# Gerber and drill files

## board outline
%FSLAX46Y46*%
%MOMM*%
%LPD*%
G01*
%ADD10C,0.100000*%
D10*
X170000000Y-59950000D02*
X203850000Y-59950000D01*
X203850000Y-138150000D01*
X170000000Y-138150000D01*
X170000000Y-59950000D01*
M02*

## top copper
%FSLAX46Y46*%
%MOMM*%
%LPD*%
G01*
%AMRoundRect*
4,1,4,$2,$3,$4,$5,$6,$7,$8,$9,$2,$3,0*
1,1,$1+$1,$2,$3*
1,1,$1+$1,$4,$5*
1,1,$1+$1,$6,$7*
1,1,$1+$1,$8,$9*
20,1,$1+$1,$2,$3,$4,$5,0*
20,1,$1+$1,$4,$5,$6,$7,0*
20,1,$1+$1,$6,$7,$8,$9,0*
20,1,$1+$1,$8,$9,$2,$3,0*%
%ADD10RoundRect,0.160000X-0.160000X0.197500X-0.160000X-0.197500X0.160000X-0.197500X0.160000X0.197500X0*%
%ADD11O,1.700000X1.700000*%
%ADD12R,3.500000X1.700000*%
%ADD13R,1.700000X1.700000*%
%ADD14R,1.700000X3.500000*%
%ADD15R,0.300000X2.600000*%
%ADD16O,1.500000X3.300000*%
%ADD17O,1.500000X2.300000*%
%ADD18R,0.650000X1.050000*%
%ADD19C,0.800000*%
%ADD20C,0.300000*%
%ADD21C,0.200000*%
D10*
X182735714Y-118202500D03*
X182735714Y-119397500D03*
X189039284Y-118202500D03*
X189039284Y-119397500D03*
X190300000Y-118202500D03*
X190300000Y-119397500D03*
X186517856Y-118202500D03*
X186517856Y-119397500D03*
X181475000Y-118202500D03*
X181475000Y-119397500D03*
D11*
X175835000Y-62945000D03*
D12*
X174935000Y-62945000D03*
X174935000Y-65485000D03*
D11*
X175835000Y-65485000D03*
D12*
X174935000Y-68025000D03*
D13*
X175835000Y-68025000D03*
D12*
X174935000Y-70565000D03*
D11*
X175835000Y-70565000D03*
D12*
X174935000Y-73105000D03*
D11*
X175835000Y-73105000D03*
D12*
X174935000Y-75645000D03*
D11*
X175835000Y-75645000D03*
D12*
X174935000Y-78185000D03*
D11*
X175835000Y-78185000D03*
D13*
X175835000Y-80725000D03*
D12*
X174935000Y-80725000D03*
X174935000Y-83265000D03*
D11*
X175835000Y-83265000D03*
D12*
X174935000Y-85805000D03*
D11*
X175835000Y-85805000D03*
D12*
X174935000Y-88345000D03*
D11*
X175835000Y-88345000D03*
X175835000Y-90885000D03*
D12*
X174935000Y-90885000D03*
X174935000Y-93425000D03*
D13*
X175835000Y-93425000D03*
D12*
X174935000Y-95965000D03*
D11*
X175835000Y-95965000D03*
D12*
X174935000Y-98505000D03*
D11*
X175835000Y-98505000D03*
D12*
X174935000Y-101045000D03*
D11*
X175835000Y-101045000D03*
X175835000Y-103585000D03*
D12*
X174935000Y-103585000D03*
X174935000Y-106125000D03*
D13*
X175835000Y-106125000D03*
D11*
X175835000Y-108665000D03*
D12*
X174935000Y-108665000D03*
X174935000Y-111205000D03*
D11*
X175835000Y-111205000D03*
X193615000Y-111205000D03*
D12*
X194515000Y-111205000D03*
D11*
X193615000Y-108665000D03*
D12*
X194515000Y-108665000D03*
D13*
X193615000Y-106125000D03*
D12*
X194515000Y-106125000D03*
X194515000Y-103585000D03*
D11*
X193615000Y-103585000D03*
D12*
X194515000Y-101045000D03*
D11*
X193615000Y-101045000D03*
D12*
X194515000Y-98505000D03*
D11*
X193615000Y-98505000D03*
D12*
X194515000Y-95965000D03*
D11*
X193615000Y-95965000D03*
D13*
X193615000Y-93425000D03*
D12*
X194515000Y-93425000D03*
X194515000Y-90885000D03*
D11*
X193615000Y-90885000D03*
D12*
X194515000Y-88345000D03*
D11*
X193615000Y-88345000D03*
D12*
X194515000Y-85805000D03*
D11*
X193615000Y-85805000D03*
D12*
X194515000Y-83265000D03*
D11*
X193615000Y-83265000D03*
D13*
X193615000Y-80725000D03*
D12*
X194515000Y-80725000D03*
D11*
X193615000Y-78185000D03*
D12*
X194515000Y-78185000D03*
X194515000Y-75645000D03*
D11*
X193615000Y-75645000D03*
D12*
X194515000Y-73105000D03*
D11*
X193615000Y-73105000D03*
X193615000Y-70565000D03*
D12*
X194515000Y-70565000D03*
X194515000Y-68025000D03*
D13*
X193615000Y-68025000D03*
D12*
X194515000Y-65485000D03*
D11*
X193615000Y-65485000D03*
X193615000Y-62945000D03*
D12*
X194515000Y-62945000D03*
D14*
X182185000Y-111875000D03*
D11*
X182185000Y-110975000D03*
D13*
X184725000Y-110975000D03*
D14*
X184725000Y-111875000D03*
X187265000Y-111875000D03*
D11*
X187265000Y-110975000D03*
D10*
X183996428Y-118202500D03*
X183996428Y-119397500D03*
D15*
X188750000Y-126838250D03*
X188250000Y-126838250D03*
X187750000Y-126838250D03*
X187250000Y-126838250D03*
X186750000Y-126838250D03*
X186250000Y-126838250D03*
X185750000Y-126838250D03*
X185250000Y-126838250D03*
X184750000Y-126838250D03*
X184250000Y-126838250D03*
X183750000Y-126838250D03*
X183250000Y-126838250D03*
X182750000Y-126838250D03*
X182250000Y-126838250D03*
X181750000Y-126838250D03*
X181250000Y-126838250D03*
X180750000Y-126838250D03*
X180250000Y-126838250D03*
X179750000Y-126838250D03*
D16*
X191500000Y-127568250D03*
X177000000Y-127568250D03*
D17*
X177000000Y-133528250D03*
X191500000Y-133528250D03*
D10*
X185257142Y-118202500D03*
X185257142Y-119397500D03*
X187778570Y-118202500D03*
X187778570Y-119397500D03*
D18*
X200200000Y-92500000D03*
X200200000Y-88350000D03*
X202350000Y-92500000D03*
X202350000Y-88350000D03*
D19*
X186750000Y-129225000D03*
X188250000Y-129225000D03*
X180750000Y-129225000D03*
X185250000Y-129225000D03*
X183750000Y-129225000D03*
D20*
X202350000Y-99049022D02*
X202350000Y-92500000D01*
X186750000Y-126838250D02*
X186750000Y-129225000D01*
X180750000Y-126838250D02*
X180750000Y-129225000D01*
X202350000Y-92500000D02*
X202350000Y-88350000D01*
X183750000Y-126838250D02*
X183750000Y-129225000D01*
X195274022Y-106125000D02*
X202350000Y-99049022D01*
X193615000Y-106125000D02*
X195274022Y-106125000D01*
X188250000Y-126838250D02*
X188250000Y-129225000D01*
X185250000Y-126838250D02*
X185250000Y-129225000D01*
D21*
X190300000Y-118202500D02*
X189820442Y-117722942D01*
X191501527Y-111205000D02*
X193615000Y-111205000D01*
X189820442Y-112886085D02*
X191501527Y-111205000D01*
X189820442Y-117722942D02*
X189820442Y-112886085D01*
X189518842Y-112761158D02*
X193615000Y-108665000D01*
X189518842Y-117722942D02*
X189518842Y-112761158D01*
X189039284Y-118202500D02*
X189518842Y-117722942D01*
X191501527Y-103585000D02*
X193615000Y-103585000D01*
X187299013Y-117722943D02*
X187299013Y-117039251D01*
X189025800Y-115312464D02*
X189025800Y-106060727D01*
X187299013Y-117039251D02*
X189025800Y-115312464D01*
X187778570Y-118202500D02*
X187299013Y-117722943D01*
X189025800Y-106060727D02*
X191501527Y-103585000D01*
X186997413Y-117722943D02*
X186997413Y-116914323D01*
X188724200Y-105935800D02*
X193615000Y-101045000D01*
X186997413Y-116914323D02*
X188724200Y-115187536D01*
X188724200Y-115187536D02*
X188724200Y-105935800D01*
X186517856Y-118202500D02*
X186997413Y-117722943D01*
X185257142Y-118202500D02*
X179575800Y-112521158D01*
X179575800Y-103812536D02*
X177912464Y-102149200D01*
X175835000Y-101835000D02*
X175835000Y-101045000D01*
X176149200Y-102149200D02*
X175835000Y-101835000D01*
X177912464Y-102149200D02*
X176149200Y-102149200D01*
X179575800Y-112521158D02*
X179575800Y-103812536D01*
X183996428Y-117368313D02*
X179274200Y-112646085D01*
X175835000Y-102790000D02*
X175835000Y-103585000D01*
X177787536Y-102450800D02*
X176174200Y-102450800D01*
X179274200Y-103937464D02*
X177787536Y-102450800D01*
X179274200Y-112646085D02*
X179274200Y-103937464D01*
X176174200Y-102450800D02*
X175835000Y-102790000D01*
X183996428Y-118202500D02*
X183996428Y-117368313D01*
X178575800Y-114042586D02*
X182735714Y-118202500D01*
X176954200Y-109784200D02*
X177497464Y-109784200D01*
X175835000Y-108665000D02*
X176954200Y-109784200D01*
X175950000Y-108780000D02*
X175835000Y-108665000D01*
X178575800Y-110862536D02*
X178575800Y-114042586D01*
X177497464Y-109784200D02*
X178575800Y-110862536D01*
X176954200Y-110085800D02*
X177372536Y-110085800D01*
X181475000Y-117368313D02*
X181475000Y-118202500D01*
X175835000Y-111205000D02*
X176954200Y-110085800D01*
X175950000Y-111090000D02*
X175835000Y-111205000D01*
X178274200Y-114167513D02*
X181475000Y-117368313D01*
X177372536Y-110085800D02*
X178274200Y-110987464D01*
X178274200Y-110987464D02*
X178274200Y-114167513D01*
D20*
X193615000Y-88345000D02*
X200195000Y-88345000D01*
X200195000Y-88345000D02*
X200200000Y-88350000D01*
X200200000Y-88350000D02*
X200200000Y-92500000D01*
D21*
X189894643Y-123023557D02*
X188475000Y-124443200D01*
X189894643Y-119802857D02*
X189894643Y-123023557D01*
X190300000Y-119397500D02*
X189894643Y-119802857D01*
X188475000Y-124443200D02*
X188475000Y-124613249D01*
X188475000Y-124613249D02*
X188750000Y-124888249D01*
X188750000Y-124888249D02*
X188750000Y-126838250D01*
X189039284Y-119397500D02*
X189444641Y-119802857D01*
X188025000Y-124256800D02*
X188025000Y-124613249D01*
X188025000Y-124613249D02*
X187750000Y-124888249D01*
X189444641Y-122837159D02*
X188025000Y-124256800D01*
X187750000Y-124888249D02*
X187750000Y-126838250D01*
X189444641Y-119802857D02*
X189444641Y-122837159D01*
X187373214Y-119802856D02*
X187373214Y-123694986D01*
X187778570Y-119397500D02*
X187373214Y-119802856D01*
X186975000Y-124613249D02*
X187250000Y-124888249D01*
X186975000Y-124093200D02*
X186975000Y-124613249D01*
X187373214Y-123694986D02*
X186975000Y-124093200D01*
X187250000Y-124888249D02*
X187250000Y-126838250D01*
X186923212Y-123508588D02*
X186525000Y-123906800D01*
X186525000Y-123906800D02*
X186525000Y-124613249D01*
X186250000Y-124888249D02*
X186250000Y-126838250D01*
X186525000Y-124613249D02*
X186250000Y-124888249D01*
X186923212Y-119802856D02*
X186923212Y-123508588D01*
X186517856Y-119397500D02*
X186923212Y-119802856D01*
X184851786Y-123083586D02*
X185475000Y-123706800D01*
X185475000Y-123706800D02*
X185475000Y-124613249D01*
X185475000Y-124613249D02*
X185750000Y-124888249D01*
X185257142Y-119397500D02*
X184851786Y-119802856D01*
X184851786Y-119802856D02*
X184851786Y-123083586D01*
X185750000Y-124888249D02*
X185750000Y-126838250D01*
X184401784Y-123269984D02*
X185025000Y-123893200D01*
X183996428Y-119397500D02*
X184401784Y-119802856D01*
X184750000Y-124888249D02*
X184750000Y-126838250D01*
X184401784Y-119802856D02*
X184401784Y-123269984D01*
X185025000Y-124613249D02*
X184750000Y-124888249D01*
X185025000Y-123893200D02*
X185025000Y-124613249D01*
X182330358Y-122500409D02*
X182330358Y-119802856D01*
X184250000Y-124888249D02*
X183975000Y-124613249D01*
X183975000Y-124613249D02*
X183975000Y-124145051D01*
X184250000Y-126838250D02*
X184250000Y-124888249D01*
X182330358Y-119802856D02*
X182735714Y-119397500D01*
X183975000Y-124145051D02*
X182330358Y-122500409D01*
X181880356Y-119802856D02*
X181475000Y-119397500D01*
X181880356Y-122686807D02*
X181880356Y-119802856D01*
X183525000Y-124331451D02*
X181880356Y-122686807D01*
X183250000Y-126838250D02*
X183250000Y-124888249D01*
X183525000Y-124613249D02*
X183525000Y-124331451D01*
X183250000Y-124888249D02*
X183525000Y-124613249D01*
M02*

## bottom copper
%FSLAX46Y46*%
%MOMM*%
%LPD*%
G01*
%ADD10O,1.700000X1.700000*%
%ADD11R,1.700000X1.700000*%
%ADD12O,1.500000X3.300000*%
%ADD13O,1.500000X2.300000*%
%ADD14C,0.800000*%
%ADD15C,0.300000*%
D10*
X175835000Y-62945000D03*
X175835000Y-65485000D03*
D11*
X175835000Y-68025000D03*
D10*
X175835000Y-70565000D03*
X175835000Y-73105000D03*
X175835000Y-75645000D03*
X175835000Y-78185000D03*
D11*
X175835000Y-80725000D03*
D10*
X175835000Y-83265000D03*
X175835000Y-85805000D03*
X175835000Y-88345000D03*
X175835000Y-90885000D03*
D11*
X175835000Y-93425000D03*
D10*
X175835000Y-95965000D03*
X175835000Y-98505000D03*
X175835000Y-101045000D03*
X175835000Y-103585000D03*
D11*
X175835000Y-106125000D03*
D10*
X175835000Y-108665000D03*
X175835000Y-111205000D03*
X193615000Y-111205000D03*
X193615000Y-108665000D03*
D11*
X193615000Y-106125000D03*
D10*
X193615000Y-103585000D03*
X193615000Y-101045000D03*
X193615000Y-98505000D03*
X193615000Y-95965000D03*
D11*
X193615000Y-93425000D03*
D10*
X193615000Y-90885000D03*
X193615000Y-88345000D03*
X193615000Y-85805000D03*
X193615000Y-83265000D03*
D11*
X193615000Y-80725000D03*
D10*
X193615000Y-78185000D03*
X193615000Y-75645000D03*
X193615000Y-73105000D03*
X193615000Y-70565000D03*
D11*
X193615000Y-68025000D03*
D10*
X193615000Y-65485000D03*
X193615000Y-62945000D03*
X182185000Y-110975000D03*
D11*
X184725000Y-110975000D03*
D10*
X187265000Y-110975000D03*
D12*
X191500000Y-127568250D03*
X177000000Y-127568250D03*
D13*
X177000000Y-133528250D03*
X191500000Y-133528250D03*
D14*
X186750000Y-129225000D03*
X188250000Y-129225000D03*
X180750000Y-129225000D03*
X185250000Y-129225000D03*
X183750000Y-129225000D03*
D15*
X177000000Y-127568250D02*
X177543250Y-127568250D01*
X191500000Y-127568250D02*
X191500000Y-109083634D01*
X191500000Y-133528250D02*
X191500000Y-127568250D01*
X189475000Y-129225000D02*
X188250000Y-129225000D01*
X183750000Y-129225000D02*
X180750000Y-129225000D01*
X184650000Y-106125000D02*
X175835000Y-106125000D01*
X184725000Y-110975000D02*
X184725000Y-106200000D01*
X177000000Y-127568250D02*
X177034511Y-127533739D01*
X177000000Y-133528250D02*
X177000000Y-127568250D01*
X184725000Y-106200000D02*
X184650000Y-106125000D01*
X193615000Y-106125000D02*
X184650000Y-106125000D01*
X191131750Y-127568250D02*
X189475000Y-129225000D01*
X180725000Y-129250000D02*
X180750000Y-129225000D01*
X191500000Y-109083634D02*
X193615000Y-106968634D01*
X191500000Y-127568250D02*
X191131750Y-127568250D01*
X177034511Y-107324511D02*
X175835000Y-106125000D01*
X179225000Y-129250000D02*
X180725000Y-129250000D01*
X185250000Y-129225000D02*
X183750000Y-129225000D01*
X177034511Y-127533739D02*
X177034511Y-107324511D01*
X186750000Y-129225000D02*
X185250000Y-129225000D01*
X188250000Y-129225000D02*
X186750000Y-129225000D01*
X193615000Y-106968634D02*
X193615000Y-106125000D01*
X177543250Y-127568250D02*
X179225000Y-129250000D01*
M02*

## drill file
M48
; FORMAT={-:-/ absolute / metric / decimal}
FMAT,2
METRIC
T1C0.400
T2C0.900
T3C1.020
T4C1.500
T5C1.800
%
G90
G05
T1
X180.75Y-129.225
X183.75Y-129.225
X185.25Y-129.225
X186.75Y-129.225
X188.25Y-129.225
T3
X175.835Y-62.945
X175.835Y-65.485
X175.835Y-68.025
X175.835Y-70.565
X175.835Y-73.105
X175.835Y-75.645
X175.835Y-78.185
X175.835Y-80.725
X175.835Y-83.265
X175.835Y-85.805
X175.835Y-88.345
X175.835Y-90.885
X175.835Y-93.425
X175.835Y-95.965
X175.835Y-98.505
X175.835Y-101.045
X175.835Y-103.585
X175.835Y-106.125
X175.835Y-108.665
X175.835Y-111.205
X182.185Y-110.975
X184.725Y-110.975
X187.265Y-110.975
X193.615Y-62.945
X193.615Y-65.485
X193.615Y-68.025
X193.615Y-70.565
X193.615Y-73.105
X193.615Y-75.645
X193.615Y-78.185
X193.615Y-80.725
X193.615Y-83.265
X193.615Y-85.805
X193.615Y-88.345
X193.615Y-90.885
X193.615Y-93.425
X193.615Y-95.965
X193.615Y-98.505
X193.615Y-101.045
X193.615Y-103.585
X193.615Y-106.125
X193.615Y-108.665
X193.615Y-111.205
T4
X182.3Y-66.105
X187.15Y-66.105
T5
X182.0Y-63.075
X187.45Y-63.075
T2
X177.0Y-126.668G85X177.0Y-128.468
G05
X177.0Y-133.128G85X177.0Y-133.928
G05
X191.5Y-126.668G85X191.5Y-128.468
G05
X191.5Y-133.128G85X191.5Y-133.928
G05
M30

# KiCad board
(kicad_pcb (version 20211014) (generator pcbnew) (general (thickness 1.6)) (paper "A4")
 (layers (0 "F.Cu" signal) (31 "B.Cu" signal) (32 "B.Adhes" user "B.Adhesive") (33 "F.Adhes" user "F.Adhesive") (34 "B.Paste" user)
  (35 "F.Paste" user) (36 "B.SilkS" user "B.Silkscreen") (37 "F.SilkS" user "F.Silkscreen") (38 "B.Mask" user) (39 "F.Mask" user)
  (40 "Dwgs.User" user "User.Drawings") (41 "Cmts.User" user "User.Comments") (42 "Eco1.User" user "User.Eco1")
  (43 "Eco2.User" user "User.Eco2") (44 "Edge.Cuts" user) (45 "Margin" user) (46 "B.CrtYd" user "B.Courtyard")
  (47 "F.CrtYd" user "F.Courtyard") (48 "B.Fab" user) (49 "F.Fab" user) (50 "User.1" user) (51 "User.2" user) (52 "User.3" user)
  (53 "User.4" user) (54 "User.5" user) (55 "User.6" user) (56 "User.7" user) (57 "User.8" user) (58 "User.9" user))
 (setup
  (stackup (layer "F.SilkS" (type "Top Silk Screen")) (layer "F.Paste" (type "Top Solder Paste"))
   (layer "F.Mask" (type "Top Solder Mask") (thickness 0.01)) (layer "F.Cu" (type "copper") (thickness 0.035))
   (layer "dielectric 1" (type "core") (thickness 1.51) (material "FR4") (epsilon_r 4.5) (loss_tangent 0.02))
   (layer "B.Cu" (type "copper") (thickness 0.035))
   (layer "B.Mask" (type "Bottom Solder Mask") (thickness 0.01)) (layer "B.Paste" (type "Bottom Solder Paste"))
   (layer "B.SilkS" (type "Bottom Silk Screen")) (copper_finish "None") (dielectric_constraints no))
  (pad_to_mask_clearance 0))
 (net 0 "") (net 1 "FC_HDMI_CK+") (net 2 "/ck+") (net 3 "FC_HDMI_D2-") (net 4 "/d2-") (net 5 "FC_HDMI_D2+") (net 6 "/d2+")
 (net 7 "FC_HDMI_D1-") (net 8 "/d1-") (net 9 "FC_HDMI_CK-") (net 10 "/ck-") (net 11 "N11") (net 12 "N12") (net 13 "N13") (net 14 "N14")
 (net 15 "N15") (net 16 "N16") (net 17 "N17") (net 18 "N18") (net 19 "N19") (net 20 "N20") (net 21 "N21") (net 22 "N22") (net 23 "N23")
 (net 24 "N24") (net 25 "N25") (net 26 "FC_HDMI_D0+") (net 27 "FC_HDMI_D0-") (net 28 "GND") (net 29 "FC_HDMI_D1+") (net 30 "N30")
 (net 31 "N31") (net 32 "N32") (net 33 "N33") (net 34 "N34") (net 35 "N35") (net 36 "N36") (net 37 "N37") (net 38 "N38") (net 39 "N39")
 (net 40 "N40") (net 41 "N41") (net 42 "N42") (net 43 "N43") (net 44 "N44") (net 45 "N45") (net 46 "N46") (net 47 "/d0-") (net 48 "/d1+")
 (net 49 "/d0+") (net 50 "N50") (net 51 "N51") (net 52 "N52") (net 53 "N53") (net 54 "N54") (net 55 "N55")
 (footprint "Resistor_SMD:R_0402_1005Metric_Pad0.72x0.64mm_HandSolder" (layer "F.Cu") (at 182.735714 118.8 -90)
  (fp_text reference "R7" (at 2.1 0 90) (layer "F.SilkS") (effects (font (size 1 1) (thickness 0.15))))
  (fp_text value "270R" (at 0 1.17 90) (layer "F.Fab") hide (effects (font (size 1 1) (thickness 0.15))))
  (pad "1" smd roundrect locked (at -0.5975 0 270) (size 0.715 0.64) (layers "F.Cu" "F.Paste" "F.Mask") (roundrect_rratio 0.25)
   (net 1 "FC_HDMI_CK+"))
  (pad "2" smd roundrect locked (at 0.5975 0 270) (size 0.715 0.64) (layers "F.Cu" "F.Paste" "F.Mask") (roundrect_rratio 0.25)
   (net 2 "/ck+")))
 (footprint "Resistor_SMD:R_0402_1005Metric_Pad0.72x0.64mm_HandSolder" (layer "F.Cu") (at 189.039284 118.8 -90)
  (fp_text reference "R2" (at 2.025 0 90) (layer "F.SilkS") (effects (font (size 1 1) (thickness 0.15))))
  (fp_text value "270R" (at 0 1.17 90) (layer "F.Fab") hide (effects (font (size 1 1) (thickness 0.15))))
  (pad "1" smd roundrect locked (at -0.5975 0 270) (size 0.715 0.64) (layers "F.Cu" "F.Paste" "F.Mask") (roundrect_rratio 0.25)
   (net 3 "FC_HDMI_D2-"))
  (pad "2" smd roundrect locked (at 0.5975 0 270) (size 0.715 0.64) (layers "F.Cu" "F.Paste" "F.Mask") (roundrect_rratio 0.25)
   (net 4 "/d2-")))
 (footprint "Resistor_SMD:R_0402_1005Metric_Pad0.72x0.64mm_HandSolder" (layer "F.Cu") (at 190.3 118.8 -90)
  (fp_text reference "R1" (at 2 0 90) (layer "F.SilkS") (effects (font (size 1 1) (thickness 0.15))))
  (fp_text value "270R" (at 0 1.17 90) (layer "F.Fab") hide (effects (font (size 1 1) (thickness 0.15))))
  (pad "1" smd roundrect locked (at -0.5975 0 270) (size 0.715 0.64) (layers "F.Cu" "F.Paste" "F.Mask") (roundrect_rratio 0.25)
   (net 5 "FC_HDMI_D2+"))
  (pad "2" smd roundrect locked (at 0.5975 0 270) (size 0.715 0.64) (layers "F.Cu" "F.Paste" "F.Mask") (roundrect_rratio 0.25)
   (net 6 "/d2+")))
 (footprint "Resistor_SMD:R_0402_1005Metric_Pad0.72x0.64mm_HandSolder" (layer "F.Cu") (at 186.517856 118.8 -90)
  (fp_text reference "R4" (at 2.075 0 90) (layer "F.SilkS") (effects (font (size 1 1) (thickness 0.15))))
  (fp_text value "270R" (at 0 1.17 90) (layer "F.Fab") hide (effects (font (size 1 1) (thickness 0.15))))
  (pad "1" smd roundrect locked (at -0.5975 0 270) (size 0.715 0.64) (layers "F.Cu" "F.Paste" "F.Mask") (roundrect_rratio 0.25)
   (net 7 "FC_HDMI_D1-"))
  (pad "2" smd roundrect locked (at 0.5975 0 270) (size 0.715 0.64) (layers "F.Cu" "F.Paste" "F.Mask") (roundrect_rratio 0.25)
   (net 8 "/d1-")))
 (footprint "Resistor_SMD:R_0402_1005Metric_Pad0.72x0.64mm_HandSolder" (layer "F.Cu") (at 181.475 118.8 -90)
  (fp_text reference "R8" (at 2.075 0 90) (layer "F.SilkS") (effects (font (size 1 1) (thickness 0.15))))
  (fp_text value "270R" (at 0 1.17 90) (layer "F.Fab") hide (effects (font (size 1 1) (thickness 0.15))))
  (pad "1" smd roundrect locked (at -0.5975 0 270) (size 0.715 0.64) (layers "F.Cu" "F.Paste" "F.Mask") (roundrect_rratio 0.25)
   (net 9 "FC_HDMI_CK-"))
  (pad "2" smd roundrect locked (at 0.5975 0 270) (size 0.715 0.64) (layers "F.Cu" "F.Paste" "F.Mask") (roundrect_rratio 0.25)
   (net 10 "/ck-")))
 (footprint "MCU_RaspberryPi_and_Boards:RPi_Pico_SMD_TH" (layer "F.Cu") (at 184.725 87.075)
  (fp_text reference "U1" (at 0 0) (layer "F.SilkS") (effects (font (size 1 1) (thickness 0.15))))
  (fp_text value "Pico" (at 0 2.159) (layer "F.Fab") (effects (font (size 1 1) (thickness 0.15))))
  (pad "" np_thru_hole oval locked (at -2.725 -24) (size 1.8 1.8) (drill 1.8) (layers *.Cu *.Mask))
  (pad "" np_thru_hole oval locked (at 2.725 -24) (size 1.8 1.8) (drill 1.8) (layers *.Cu *.Mask))
  (pad "" np_thru_hole oval locked (at 2.425 -20.97) (size 1.5 1.5) (drill 1.5) (layers *.Cu *.Mask))
  (pad "" np_thru_hole oval locked (at -2.425 -20.97) (size 1.5 1.5) (drill 1.5) (layers *.Cu *.Mask))
  (pad "1" thru_hole oval locked (at -8.89 -24.13) (size 1.7 1.7) (drill 1.02) (layers *.Cu *.Mask) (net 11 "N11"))
  (pad "1" smd rect locked (at -8.89 -24.13) (size 3.5 1.7) (drill (offset -0.9 0)) (layers "F.Cu" "F.Mask") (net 11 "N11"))
  (pad "2" smd rect locked (at -8.89 -21.59) (size 3.5 1.7) (drill (offset -0.9 0)) (layers "F.Cu" "F.Mask") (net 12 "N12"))
  (pad "2" thru_hole oval locked (at -8.89 -21.59) (size 1.7 1.7) (drill 1.02) (layers *.Cu *.Mask) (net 12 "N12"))
  (pad "3" smd rect locked (at -8.89 -19.05) (size 3.5 1.7) (drill (offset -0.9 0)) (layers "F.Cu" "F.Mask") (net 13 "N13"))
  (pad "3" thru_hole rect locked (at -8.89 -19.05) (size 1.7 1.7) (drill 1.02) (layers *.Cu *.Mask) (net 13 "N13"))
  (pad "4" smd rect locked (at -8.89 -16.51) (size 3.5 1.7) (drill (offset -0.9 0)) (layers "F.Cu" "F.Mask") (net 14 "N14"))
  (pad "4" thru_hole oval locked (at -8.89 -16.51) (size 1.7 1.7) (drill 1.02) (layers *.Cu *.Mask) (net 14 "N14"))
  (pad "5" smd rect locked (at -8.89 -13.97) (size 3.5 1.7) (drill (offset -0.9 0)) (layers "F.Cu" "F.Mask") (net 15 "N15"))
  (pad "5" thru_hole oval locked (at -8.89 -13.97) (size 1.7 1.7) (drill 1.02) (layers *.Cu *.Mask) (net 15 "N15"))
  (pad "6" smd rect locked (at -8.89 -11.43) (size 3.5 1.7) (drill (offset -0.9 0)) (layers "F.Cu" "F.Mask") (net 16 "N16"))
  (pad "6" thru_hole oval locked (at -8.89 -11.43) (size 1.7 1.7) (drill 1.02) (layers *.Cu *.Mask) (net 16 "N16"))
  (pad "7" smd rect locked (at -8.89 -8.89) (size 3.5 1.7) (drill (offset -0.9 0)) (layers "F.Cu" "F.Mask") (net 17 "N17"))
  (pad "7" thru_hole oval locked (at -8.89 -8.89) (size 1.7 1.7) (drill 1.02) (layers *.Cu *.Mask) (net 17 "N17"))
  (pad "8" thru_hole rect locked (at -8.89 -6.35) (size 1.7 1.7) (drill 1.02) (layers *.Cu *.Mask) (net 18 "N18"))
  (pad "8" smd rect locked (at -8.89 -6.35) (size 3.5 1.7) (drill (offset -0.9 0)) (layers "F.Cu" "F.Mask") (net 18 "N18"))
  (pad "9" smd rect locked (at -8.89 -3.81) (size 3.5 1.7) (drill (offset -0.9 0)) (layers "F.Cu" "F.Mask") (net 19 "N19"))
  (pad "9" thru_hole oval locked (at -8.89 -3.81) (size 1.7 1.7) (drill 1.02) (layers *.Cu *.Mask) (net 19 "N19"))
  (pad "10" smd rect locked (at -8.89 -1.27) (size 3.5 1.7) (drill (offset -0.9 0)) (layers "F.Cu" "F.Mask") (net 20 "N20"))
  (pad "10" thru_hole oval locked (at -8.89 -1.27) (size 1.7 1.7) (drill 1.02) (layers *.Cu *.Mask) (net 20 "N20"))
  (pad "11" smd rect locked (at -8.89 1.27) (size 3.5 1.7) (drill (offset -0.9 0)) (layers "F.Cu" "F.Mask") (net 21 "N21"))
  (pad "11" thru_hole oval locked (at -8.89 1.27) (size 1.7 1.7) (drill 1.02) (layers *.Cu *.Mask) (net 21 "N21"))
  (pad "12" thru_hole oval locked (at -8.89 3.81) (size 1.7 1.7) (drill 1.02) (layers *.Cu *.Mask) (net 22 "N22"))
  (pad "12" smd rect locked (at -8.89 3.81) (size 3.5 1.7) (drill (offset -0.9 0)) (layers "F.Cu" "F.Mask") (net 22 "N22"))
  (pad "13" smd rect locked (at -8.89 6.35) (size 3.5 1.7) (drill (offset -0.9 0)) (layers "F.Cu" "F.Mask") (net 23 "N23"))
  (pad "13" thru_hole rect locked (at -8.89 6.35) (size 1.7 1.7) (drill 1.02) (layers *.Cu *.Mask) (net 23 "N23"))
  (pad "14" smd rect locked (at -8.89 8.89) (size 3.5 1.7) (drill (offset -0.9 0)) (layers "F.Cu" "F.Mask") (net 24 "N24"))
  (pad "14" thru_hole oval locked (at -8.89 8.89) (size 1.7 1.7) (drill 1.02) (layers *.Cu *.Mask) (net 24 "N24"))
  (pad "15" smd rect locked (at -8.89 11.43) (size 3.5 1.7) (drill (offset -0.9 0)) (layers "F.Cu" "F.Mask") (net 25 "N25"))
  (pad "15" thru_hole oval locked (at -8.89 11.43) (size 1.7 1.7) (drill 1.02) (layers *.Cu *.Mask) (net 25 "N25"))
  (pad "16" smd rect locked (at -8.89 13.97) (size 3.5 1.7) (drill (offset -0.9 0)) (layers "F.Cu" "F.Mask") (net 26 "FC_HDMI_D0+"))
  (pad "16" thru_hole oval locked (at -8.89 13.97) (size 1.7 1.7) (drill 1.02) (layers *.Cu *.Mask) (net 26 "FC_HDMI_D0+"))
  (pad "17" thru_hole oval locked (at -8.89 16.51) (size 1.7 1.7) (drill 1.02) (layers *.Cu *.Mask) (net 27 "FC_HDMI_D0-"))
  (pad "17" smd rect locked (at -8.89 16.51) (size 3.5 1.7) (drill (offset -0.9 0)) (layers "F.Cu" "F.Mask") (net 27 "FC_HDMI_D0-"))
  (pad "18" smd rect locked (at -8.89 19.05) (size 3.5 1.7) (drill (offset -0.9 0)) (layers "F.Cu" "F.Mask") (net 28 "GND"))
  (pad "18" thru_hole rect locked (at -8.89 19.05) (size 1.7 1.7) (drill 1.02) (layers *.Cu *.Mask) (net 28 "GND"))
  (pad "19" thru_hole oval locked (at -8.89 21.59) (size 1.7 1.7) (drill 1.02) (layers *.Cu *.Mask) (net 1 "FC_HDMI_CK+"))
  (pad "19" smd rect locked (at -8.89 21.59) (size 3.5 1.7) (drill (offset -0.9 0)) (layers "F.Cu" "F.Mask") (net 1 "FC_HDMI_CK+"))
  (pad "20" smd rect locked (at -8.89 24.13) (size 3.5 1.7) (drill (offset -0.9 0)) (layers "F.Cu" "F.Mask") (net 9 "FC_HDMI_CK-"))
  (pad "20" thru_hole oval locked (at -8.89 24.13) (size 1.7 1.7) (drill 1.02) (layers *.Cu *.Mask) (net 9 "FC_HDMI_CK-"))
  (pad "21" thru_hole oval locked (at 8.89 24.13) (size 1.7 1.7) (drill 1.02) (layers *.Cu *.Mask) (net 5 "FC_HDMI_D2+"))
  (pad "21" smd rect locked (at 8.89 24.13) (size 3.5 1.7) (drill (offset 0.9 0)) (layers "F.Cu" "F.Mask") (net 5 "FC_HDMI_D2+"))
  (pad "22" thru_hole oval locked (at 8.89 21.59) (size 1.7 1.7) (drill 1.02) (layers *.Cu *.Mask) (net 3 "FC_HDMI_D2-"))
  (pad "22" smd rect locked (at 8.89 21.59) (size 3.5 1.7) (drill (offset 0.9 0)) (layers "F.Cu" "F.Mask") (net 3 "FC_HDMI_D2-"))
  (pad "23" thru_hole rect locked (at 8.89 19.05) (size 1.7 1.7) (drill 1.02) (layers *.Cu *.Mask) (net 28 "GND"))
  (pad "23" smd rect locked (at 8.89 19.05) (size 3.5 1.7) (drill (offset 0.9 0)) (layers "F.Cu" "F.Mask") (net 28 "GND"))
  (pad "24" smd rect locked (at 8.89 16.51) (size 3.5 1.7) (drill (offset 0.9 0)) (layers "F.Cu" "F.Mask") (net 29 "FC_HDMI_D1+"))
  (pad "24" thru_hole oval locked (at 8.89 16.51) (size 1.7 1.7) (drill 1.02) (layers *.Cu *.Mask) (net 29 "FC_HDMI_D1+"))
  (pad "25" smd rect locked (at 8.89 13.97) (size 3.5 1.7) (drill (offset 0.9 0)) (layers "F.Cu" "F.Mask") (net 7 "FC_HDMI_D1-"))
  (pad "25" thru_hole oval locked (at 8.89 13.97) (size 1.7 1.7) (drill 1.02) (layers *.Cu *.Mask) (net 7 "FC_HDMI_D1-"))
  (pad "26" smd rect locked (at 8.89 11.43) (size 3.5 1.7) (drill (offset 0.9 0)) (layers "F.Cu" "F.Mask") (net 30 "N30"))
  (pad "26" thru_hole oval locked (at 8.89 11.43) (size 1.7 1.7) (drill 1.02) (layers *.Cu *.Mask) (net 30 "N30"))
  (pad "27" smd rect locked (at 8.89 8.89) (size 3.5 1.7) (drill (offset 0.9 0)) (layers "F.Cu" "F.Mask") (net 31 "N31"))
  (pad "27" thru_hole oval locked (at 8.89 8.89) (size 1.7 1.7) (drill 1.02) (layers *.Cu *.Mask) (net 31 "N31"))
  (pad "28" thru_hole rect locked (at 8.89 6.35) (size 1.7 1.7) (drill 1.02) (layers *.Cu *.Mask) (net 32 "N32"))
  (pad "28" smd rect locked (at 8.89 6.35) (size 3.5 1.7) (drill (offset 0.9 0)) (layers "F.Cu" "F.Mask") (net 32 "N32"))
  (pad "29" smd rect locked (at 8.89 3.81) (size 3.5 1.7) (drill (offset 0.9 0)) (layers "F.Cu" "F.Mask") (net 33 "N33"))
  (pad "29" thru_hole oval locked (at 8.89 3.81) (size 1.7 1.7) (drill 1.02) (layers *.Cu *.Mask) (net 33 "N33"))
  (pad "30" smd rect locked (at 8.89 1.27) (size 3.5 1.7) (drill (offset 0.9 0)) (layers "F.Cu" "F.Mask") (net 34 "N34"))
  (pad "30" thru_hole oval locked (at 8.89 1.27) (size 1.7 1.7) (drill 1.02) (layers *.Cu *.Mask) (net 34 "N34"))
  (pad "31" smd rect locked (at 8.89 -1.27) (size 3.5 1.7) (drill (offset 0.9 0)) (layers "F.Cu" "F.Mask") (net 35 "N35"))
  (pad "31" thru_hole oval locked (at 8.89 -1.27) (size 1.7 1.7) (drill 1.02) (layers *.Cu *.Mask) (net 35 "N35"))
  (pad "32" smd rect locked (at 8.89 -3.81) (size 3.5 1.7) (drill (offset 0.9 0)) (layers "F.Cu" "F.Mask") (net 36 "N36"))
  (pad "32" thru_hole oval locked (at 8.89 -3.81) (size 1.7 1.7) (drill 1.02) (layers *.Cu *.Mask) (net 36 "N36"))
  (pad "33" thru_hole rect locked (at 8.89 -6.35) (size 1.7 1.7) (drill 1.02) (layers *.Cu *.Mask) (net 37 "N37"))
  (pad "33" smd rect locked (at 8.89 -6.35) (size 3.5 1.7) (drill (offset 0.9 0)) (layers "F.Cu" "F.Mask") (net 37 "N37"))
  (pad "34" thru_hole oval locked (at 8.89 -8.89) (size 1.7 1.7) (drill 1.02) (layers *.Cu *.Mask) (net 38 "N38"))
  (pad "34" smd rect locked (at 8.89 -8.89) (size 3.5 1.7) (drill (offset 0.9 0)) (layers "F.Cu" "F.Mask") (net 38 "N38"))
  (pad "35" smd rect locked (at 8.89 -11.43) (size 3.5 1.7) (drill (offset 0.9 0)) (layers "F.Cu" "F.Mask") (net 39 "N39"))
  (pad "35" thru_hole oval locked (at 8.89 -11.43) (size 1.7 1.7) (drill 1.02) (layers *.Cu *.Mask) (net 39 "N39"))
  (pad "36" smd rect locked (at 8.89 -13.97) (size 3.5 1.7) (drill (offset 0.9 0)) (layers "F.Cu" "F.Mask") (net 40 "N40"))
  (pad "36" thru_hole oval locked (at 8.89 -13.97) (size 1.7 1.7) (drill 1.02) (layers *.Cu *.Mask) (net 40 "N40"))
  (pad "37" thru_hole oval locked (at 8.89 -16.51) (size 1.7 1.7) (drill 1.02) (layers *.Cu *.Mask) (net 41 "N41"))
  (pad "37" smd rect locked (at 8.89 -16.51) (size 3.5 1.7) (drill (offset 0.9 0)) (layers "F.Cu" "F.Mask") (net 41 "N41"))
  (pad "38" smd rect locked (at 8.89 -19.05) (size 3.5 1.7) (drill (offset 0.9 0)) (layers "F.Cu" "F.Mask") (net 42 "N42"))
  (pad "38" thru_hole rect locked (at 8.89 -19.05) (size 1.7 1.7) (drill 1.02) (layers *.Cu *.Mask) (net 42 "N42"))
  (pad "39" smd rect locked (at 8.89 -21.59) (size 3.5 1.7) (drill (offset 0.9 0)) (layers "F.Cu" "F.Mask") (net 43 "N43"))
  (pad "39" thru_hole oval locked (at 8.89 -21.59) (size 1.7 1.7) (drill 1.02) (layers *.Cu *.Mask) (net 43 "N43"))
  (pad "40" thru_hole oval locked (at 8.89 -24.13) (size 1.7 1.7) (drill 1.02) (layers *.Cu *.Mask) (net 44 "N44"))
  (pad "40" smd rect locked (at 8.89 -24.13) (size 3.5 1.7) (drill (offset 0.9 0)) (layers "F.Cu" "F.Mask") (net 44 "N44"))
  (pad "41" smd rect locked (at -2.54 23.9 90) (size 3.5 1.7) (drill (offset -0.9 0)) (layers "F.Cu" "F.Mask") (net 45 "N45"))
  (pad "41" thru_hole oval locked (at -2.54 23.9) (size 1.7 1.7) (drill 1.02) (layers *.Cu *.Mask) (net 45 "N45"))
  (pad "42" thru_hole rect locked (at 0 23.9) (size 1.7 1.7) (drill 1.02) (layers *.Cu *.Mask) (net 28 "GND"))
  (pad "42" smd rect locked (at 0 23.9 90) (size 3.5 1.7) (drill (offset -0.9 0)) (layers "F.Cu" "F.Mask") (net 28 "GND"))
  (pad "43" smd rect locked (at 2.54 23.9 90) (size 3.5 1.7) (drill (offset -0.9 0)) (layers "F.Cu" "F.Mask") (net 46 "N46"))
  (pad "43" thru_hole oval locked (at 2.54 23.9) (size 1.7 1.7) (drill 1.02) (layers *.Cu *.Mask) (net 46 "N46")))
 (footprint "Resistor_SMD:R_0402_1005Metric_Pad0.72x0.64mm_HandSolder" (layer "F.Cu") (at 183.996428 118.8 -90)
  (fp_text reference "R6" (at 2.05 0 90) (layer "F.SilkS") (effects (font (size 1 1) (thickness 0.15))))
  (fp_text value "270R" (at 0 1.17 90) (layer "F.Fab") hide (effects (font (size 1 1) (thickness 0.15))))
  (pad "1" smd roundrect locked (at -0.5975 0 270) (size 0.715 0.64) (layers "F.Cu" "F.Paste" "F.Mask") (roundrect_rratio 0.25)
   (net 27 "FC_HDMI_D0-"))
  (pad "2" smd roundrect locked (at 0.5975 0 270) (size 0.715 0.64) (layers "F.Cu" "F.Paste" "F.Mask") (roundrect_rratio 0.25)
   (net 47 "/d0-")))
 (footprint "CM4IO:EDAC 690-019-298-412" (layer "F.Cu") (at 184.25 127.56825)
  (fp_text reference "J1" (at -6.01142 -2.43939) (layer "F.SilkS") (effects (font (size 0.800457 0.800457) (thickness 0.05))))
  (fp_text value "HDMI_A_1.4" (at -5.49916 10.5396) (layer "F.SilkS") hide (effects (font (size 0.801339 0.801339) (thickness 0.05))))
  (pad "1" smd rect (at 4.5 -0.73 90) (size 2.6 0.3) (layers "F.Cu" "F.Paste" "F.Mask") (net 6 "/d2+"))
  (pad "2" smd rect (at 4 -0.73 90) (size 2.6 0.3) (layers "F.Cu" "F.Paste" "F.Mask") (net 28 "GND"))
  (pad "3" smd rect (at 3.5 -0.73 90) (size 2.6 0.3) (layers "F.Cu" "F.Paste" "F.Mask") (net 4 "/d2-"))
  (pad "4" smd rect (at 3 -0.73 90) (size 2.6 0.3) (layers "F.Cu" "F.Paste" "F.Mask") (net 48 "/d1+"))
  (pad "5" smd rect (at 2.5 -0.73 90) (size 2.6 0.3) (layers "F.Cu" "F.Paste" "F.Mask") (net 28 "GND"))
  (pad "6" smd rect (at 2 -0.73 90) (size 2.6 0.3) (layers "F.Cu" "F.Paste" "F.Mask") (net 8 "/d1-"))
  (pad "7" smd rect (at 1.5 -0.73 90) (size 2.6 0.3) (layers "F.Cu" "F.Paste" "F.Mask") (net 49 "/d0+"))
  (pad "8" smd rect (at 1 -0.73 90) (size 2.6 0.3) (layers "F.Cu" "F.Paste" "F.Mask") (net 28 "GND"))
  (pad "9" smd rect (at 0.5 -0.73 90) (size 2.6 0.3) (layers "F.Cu" "F.Paste" "F.Mask") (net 47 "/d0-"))
  (pad "10" smd rect (at 0 -0.73 90) (size 2.6 0.3) (layers "F.Cu" "F.Paste" "F.Mask") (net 2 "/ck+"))
  (pad "11" smd rect (at -0.5 -0.73 90) (size 2.6 0.3) (layers "F.Cu" "F.Paste" "F.Mask") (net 28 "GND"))
  (pad "12" smd rect (at -1 -0.73 90) (size 2.6 0.3) (layers "F.Cu" "F.Paste" "F.Mask") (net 10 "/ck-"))
  (pad "13" smd rect (at -1.5 -0.73 90) (size 2.6 0.3) (layers "F.Cu" "F.Paste" "F.Mask") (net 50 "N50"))
  (pad "14" smd rect (at -2 -0.73 90) (size 2.6 0.3) (layers "F.Cu" "F.Paste" "F.Mask") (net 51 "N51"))
  (pad "15" smd rect (at -2.5 -0.73 90) (size 2.6 0.3) (layers "F.Cu" "F.Paste" "F.Mask") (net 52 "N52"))
  (pad "16" smd rect (at -3 -0.73 90) (size 2.6 0.3) (layers "F.Cu" "F.Paste" "F.Mask") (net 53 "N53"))
  (pad "17" smd rect (at -3.5 -0.73 90) (size 2.6 0.3) (layers "F.Cu" "F.Paste" "F.Mask") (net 28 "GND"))
  (pad "18" smd rect (at -4 -0.73 90) (size 2.6 0.3) (layers "F.Cu" "F.Paste" "F.Mask") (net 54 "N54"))
  (pad "19" smd rect (at -4.5 -0.73 90) (size 2.6 0.3) (layers "F.Cu" "F.Paste" "F.Mask") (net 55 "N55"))
  (pad "SH1" thru_hole oval (at 7.25 0) (size 1.5 3.3) (drill oval 0.9 2.7) (layers *.Cu *.Mask) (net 28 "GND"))
  (pad "SH2" thru_hole oval (at -7.25 0) (size 1.5 3.3) (drill oval 0.9 2.7) (layers *.Cu *.Mask) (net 28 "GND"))
  (pad "SH3" thru_hole oval (at -7.25 5.96) (size 1.5 2.3) (drill oval 0.9 1.7) (layers *.Cu *.Mask) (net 28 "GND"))
  (pad "SH4" thru_hole oval (at 7.25 5.96) (size 1.5 2.3) (drill oval 0.9 1.7) (layers *.Cu *.Mask) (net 28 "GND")))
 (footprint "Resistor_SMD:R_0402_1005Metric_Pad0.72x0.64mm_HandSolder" (layer "F.Cu") (at 185.257142 118.8 -90)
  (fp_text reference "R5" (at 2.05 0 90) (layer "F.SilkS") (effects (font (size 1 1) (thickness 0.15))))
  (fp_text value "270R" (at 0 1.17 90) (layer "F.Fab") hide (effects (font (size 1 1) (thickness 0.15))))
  (pad "1" smd roundrect locked (at -0.5975 0 270) (size 0.715 0.64) (layers "F.Cu" "F.Paste" "F.Mask") (roundrect_rratio 0.25)
   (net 26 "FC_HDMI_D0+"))
  (pad "2" smd roundrect locked (at 0.5975 0 270) (size 0.715 0.64) (layers "F.Cu" "F.Paste" "F.Mask") (roundrect_rratio 0.25)
   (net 49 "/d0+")))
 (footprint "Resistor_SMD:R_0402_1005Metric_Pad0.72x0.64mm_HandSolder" (layer "F.Cu") (at 187.77857 118.8 -90)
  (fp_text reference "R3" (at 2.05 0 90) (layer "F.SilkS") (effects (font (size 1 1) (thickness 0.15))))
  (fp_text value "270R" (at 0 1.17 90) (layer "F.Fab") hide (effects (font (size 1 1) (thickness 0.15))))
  (pad "1" smd roundrect locked (at -0.5975 0 270) (size 0.715 0.64) (layers "F.Cu" "F.Paste" "F.Mask") (roundrect_rratio 0.25)
   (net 29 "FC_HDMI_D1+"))
  (pad "2" smd roundrect locked (at 0.5975 0 270) (size 0.715 0.64) (layers "F.Cu" "F.Paste" "F.Mask") (roundrect_rratio 0.25)
   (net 48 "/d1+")))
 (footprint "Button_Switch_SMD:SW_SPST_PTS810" (layer "F.Cu") (at 201.275 90.425 90)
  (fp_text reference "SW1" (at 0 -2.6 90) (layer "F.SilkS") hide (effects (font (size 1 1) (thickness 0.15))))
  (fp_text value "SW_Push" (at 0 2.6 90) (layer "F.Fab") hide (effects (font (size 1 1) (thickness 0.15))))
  (pad "1" smd rect locked (at -2.075 -1.075 90) (size 1.05 0.65) (layers "F.Cu" "F.Paste" "F.Mask") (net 34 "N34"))
  (pad "1" smd rect locked (at 2.075 -1.075 90) (size 1.05 0.65) (layers "F.Cu" "F.Paste" "F.Mask") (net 34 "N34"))
  (pad "2" smd rect locked (at -2.075 1.075 90) (size 1.05 0.65) (layers "F.Cu" "F.Paste" "F.Mask") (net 28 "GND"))
  (pad "2" smd rect locked (at 2.075 1.075 90) (size 1.05 0.65) (layers "F.Cu" "F.Paste" "F.Mask") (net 28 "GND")))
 (gr_rect (start 170 59.95) (end 203.85 138.15) (layer "Edge.Cuts") (width 0.1) (fill none))
 (segment (start 202.35 99.049022) (end 202.35 92.5) (width 0.3) (layer "F.Cu") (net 28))
 (segment (start 186.75 126.83825) (end 186.75 129.225) (width 0.3) (layer "F.Cu") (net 28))
 (segment (start 180.75 126.83825) (end 180.75 129.225) (width 0.3) (layer "F.Cu") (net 28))
 (segment (start 202.35 92.5) (end 202.35 88.35) (width 0.3) (layer "F.Cu") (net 28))
 (segment (start 183.75 126.83825) (end 183.75 129.225) (width 0.3) (layer "F.Cu") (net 28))
 (segment (start 195.274022 106.125) (end 202.35 99.049022) (width 0.3) (layer "F.Cu") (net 28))
 (segment (start 193.615 106.125) (end 195.274022 106.125) (width 0.3) (layer "F.Cu") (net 28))
 (segment (start 188.25 126.83825) (end 188.25 129.225) (width 0.3) (layer "F.Cu") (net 28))
 (segment (start 185.25 126.83825) (end 185.25 129.225) (width 0.3) (layer "F.Cu") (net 28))
 (via (at 186.75 129.225) (size 0.8) (drill 0.4) (layers "F.Cu" "B.Cu") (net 28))
 (via (at 188.25 129.225) (size 0.8) (drill 0.4) (layers "F.Cu" "B.Cu") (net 28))
 (via (at 180.75 129.225) (size 0.8) (drill 0.4) (layers "F.Cu" "B.Cu") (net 28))
 (via (at 185.25 129.225) (size 0.8) (drill 0.4) (layers "F.Cu" "B.Cu") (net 28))
 (via (at 183.75 129.225) (size 0.8) (drill 0.4) (layers "F.Cu" "B.Cu") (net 28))
 (segment (start 177 127.56825) (end 177.54325 127.56825) (width 0.3) (layer "B.Cu") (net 28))
 (segment (start 191.5 127.56825) (end 191.5 109.083634) (width 0.3) (layer "B.Cu") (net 28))
 (segment (start 191.5 133.52825) (end 191.5 127.56825) (width 0.3) (layer "B.Cu") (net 28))
 (segment (start 189.475 129.225) (end 188.25 129.225) (width 0.3) (layer "B.Cu") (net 28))
 (segment (start 183.75 129.225) (end 180.75 129.225) (width 0.3) (layer "B.Cu") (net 28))
 (segment (start 184.65 106.125) (end 175.835 106.125) (width 0.3) (layer "B.Cu") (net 28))
 (segment (start 184.725 110.975) (end 184.725 106.2) (width 0.3) (layer "B.Cu") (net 28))
 (segment (start 177 127.56825) (end 177.034511 127.533739) (width 0.3) (layer "B.Cu") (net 28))
 (segment (start 177 133.52825) (end 177 127.56825) (width 0.3) (layer "B.Cu") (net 28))
 (segment (start 184.725 106.2) (end 184.65 106.125) (width 0.3) (layer "B.Cu") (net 28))
 (segment (start 193.615 106.125) (end 184.65 106.125) (width 0.3) (layer "B.Cu") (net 28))
 (segment (start 191.13175 127.56825) (end 189.475 129.225) (width 0.3) (layer "B.Cu") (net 28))
 (segment (start 180.725 129.25) (end 180.75 129.225) (width 0.3) (layer "B.Cu") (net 28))
 (segment (start 191.5 109.083634) (end 193.615 106.968634) (width 0.3) (layer "B.Cu") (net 28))
 (segment (start 191.5 127.56825) (end 191.13175 127.56825) (width 0.3) (layer "B.Cu") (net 28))
 (segment (start 177.034511 107.324511) (end 175.835 106.125) (width 0.3) (layer "B.Cu") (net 28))
 (segment (start 179.225 129.25) (end 180.725 129.25) (width 0.3) (layer "B.Cu") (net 28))
 (segment (start 185.25 129.225) (end 183.75 129.225) (width 0.3) (layer "B.Cu") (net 28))
 (segment (start 177.034511 127.533739) (end 177.034511 107.324511) (width 0.3) (layer "B.Cu") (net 28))
 (segment (start 186.75 129.225) (end 185.25 129.225) (width 0.3) (layer "B.Cu") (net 28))
 (segment (start 188.25 129.225) (end 186.75 129.225) (width 0.3) (layer "B.Cu") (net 28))
 (segment (start 193.615 106.968634) (end 193.615 106.125) (width 0.3) (layer "B.Cu") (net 28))
 (segment (start 177.54325 127.56825) (end 179.225 129.25) (width 0.3) (layer "B.Cu") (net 28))
 (segment (start 190.3 118.2025) (end 189.820442 117.722942) (width 0.2) (layer "F.Cu") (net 5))
 (segment (start 191.501527 111.205) (end 193.615 111.205) (width 0.2) (layer "F.Cu") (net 5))
 (segment (start 189.820442 112.886085) (end 191.501527 111.205) (width 0.2) (layer "F.Cu") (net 5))
 (segment (start 189.820442 117.722942) (end 189.820442 112.886085) (width 0.2) (layer "F.Cu") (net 5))
 (segment (start 189.518842 112.761158) (end 193.615 108.665) (width 0.2) (layer "F.Cu") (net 3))
 (segment (start 189.518842 117.722942) (end 189.518842 112.761158) (width 0.2) (layer "F.Cu") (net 3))
 (segment (start 189.039284 118.2025) (end 189.518842 117.722942) (width 0.2) (layer "F.Cu") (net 3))
 (segment (start 191.501527 103.585) (end 193.615 103.585) (width 0.2) (layer "F.Cu") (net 29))
 (segment (start 187.299013 117.722943) (end 187.299013 117.039251) (width 0.2) (layer "F.Cu") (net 29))
 (segment (start 189.0258 115.312464) (end 189.0258 106.060727) (width 0.2) (layer "F.Cu") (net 29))
 (segment (start 187.299013 117.039251) (end 189.0258 115.312464) (width 0.2) (layer "F.Cu") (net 29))
 (segment (start 187.77857 118.2025) (end 187.299013 117.722943) (width 0.2) (layer "F.Cu") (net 29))
 (segment (start 189.0258 106.060727) (end 191.501527 103.585) (width 0.2) (layer "F.Cu") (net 29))
 (segment (start 186.997413 117.722943) (end 186.997413 116.914323) (width 0.2) (layer "F.Cu") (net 7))
 (segment (start 188.7242 105.9358) (end 193.615 101.045) (width 0.2) (layer "F.Cu") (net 7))
 (segment (start 186.997413 116.914323) (end 188.7242 115.187536) (width 0.2) (layer "F.Cu") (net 7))
 (segment (start 188.7242 115.187536) (end 188.7242 105.9358) (width 0.2) (layer "F.Cu") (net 7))
 (segment (start 186.517856 118.2025) (end 186.997413 117.722943) (width 0.2) (layer "F.Cu") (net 7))
 (segment (start 185.257142 118.2025) (end 179.5758 112.521158) (width 0.2) (layer "F.Cu") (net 26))
 (segment (start 179.5758 103.812536) (end 177.912464 102.1492) (width 0.2) (layer "F.Cu") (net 26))
 (segment (start 175.835 101.835) (end 175.835 101.045) (width 0.2) (layer "F.Cu") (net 26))
 (segment (start 176.1492 102.1492) (end 175.835 101.835) (width 0.2) (layer "F.Cu") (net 26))
 (segment (start 177.912464 102.1492) (end 176.1492 102.1492) (width 0.2) (layer "F.Cu") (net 26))
 (segment (start 179.5758 112.521158) (end 179.5758 103.812536) (width 0.2) (layer "F.Cu") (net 26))
 (segment (start 183.996428 117.368313) (end 179.2742 112.646085) (width 0.2) (layer "F.Cu") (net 27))
 (segment (start 175.835 102.79) (end 175.835 103.585) (width 0.2) (layer "F.Cu") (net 27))
 (segment (start 177.787536 102.4508) (end 176.1742 102.4508) (width 0.2) (layer "F.Cu") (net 27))
 (segment (start 179.2742 103.937464) (end 177.787536 102.4508) (width 0.2) (layer "F.Cu") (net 27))
 (segment (start 179.2742 112.646085) (end 179.2742 103.937464) (width 0.2) (layer "F.Cu") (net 27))
 (segment (start 176.1742 102.4508) (end 175.835 102.79) (width 0.2) (layer "F.Cu") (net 27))
 (segment (start 183.996428 118.2025) (end 183.996428 117.368313) (width 0.2) (layer "F.Cu") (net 27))
 (segment (start 178.5758 114.042586) (end 182.735714 118.2025) (width 0.2) (layer "F.Cu") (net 1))
 (segment (start 176.9542 109.7842) (end 177.497464 109.7842) (width 0.2) (layer "F.Cu") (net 1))
 (segment (start 175.835 108.665) (end 176.9542 109.7842) (width 0.2) (layer "F.Cu") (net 1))
 (segment (start 175.95 108.78) (end 175.835 108.665) (width 0.2) (layer "F.Cu") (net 1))
 (segment (start 178.5758 110.862536) (end 178.5758 114.042586) (width 0.2) (layer "F.Cu") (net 1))
 (segment (start 177.497464 109.7842) (end 178.5758 110.862536) (width 0.2) (layer "F.Cu") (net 1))
 (segment (start 176.9542 110.0858) (end 177.372536 110.0858) (width 0.2) (layer "F.Cu") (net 9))
 (segment (start 181.475 117.368313) (end 181.475 118.2025) (width 0.2) (layer "F.Cu") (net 9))
 (segment (start 175.835 111.205) (end 176.9542 110.0858) (width 0.2) (layer "F.Cu") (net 9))
 (segment (start 175.95 111.09) (end 175.835 111.205) (width 0.2) (layer "F.Cu") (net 9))
 (segment (start 178.2742 114.167513) (end 181.475 117.368313) (width 0.2) (layer "F.Cu") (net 9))
 (segment (start 177.372536 110.0858) (end 178.2742 110.987464) (width 0.2) (layer "F.Cu") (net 9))
 (segment (start 178.2742 110.987464) (end 178.2742 114.167513) (width 0.2) (layer "F.Cu") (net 9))
 (segment (start 193.615 88.345) (end 200.195 88.345) (width 0.3) (layer "F.Cu") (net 34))
 (segment (start 200.195 88.345) (end 200.2 88.35) (width 0.3) (layer "F.Cu") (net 34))
 (segment (start 200.2 88.35) (end 200.2 92.5) (width 0.3) (layer "F.Cu") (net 34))
 (segment (start 189.894643 123.023557) (end 188.475 124.4432) (width 0.2) (layer "F.Cu") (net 6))
 (segment (start 189.894643 119.802857) (end 189.894643 123.023557) (width 0.2) (layer "F.Cu") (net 6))
 (segment (start 190.3 119.3975) (end 189.894643 119.802857) (width 0.2) (layer "F.Cu") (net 6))
 (segment (start 188.475 124.4432) (end 188.475 124.613249) (width 0.2) (layer "F.Cu") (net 6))
 (segment (start 188.475 124.613249) (end 188.75 124.888249) (width 0.2) (layer "F.Cu") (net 6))
 (segment (start 188.75 124.888249) (end 188.75 126.83825) (width 0.2) (layer "F.Cu") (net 6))
 (segment (start 189.039284 119.3975) (end 189.444641 119.802857) (width 0.2) (layer "F.Cu") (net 4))
 (segment (start 188.025 124.2568) (end 188.025 124.613249) (width 0.2) (layer "F.Cu") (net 4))
 (segment (start 188.025 124.613249) (end 187.75 124.888249) (width 0.2) (layer "F.Cu") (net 4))
 (segment (start 189.444641 122.837159) (end 188.025 124.2568) (width 0.2) (layer "F.Cu") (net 4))
 (segment (start 187.75 124.888249) (end 187.75 126.83825) (width 0.2) (layer "F.Cu") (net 4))
 (segment (start 189.444641 119.802857) (end 189.444641 122.837159) (width 0.2) (layer "F.Cu") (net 4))
 (segment (start 187.373214 119.802856) (end 187.373214 123.694986) (width 0.2) (layer "F.Cu") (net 48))
 (segment (start 187.77857 119.3975) (end 187.373214 119.802856) (width 0.2) (layer "F.Cu") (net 48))
 (segment (start 186.975 124.613249) (end 187.25 124.888249) (width 0.2) (layer "F.Cu") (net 48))
 (segment (start 186.975 124.0932) (end 186.975 124.613249) (width 0.2) (layer "F.Cu") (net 48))
 (segment (start 187.373214 123.694986) (end 186.975 124.0932) (width 0.2) (layer "F.Cu") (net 48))
 (segment (start 187.25 124.888249) (end 187.25 126.83825) (width 0.2) (layer "F.Cu") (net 48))
 (segment (start 186.923212 123.508588) (end 186.525 123.9068) (width 0.2) (layer "F.Cu") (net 8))
 (segment (start 186.525 123.9068) (end 186.525 124.613249) (width 0.2) (layer "F.Cu") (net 8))
 (segment (start 186.25 124.888249) (end 186.25 126.83825) (width 0.2) (layer "F.Cu") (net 8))
 (segment (start 186.525 124.613249) (end 186.25 124.888249) (width 0.2) (layer "F.Cu") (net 8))
 (segment (start 186.923212 119.802856) (end 186.923212 123.508588) (width 0.2) (layer "F.Cu") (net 8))
 (segment (start 186.517856 119.3975) (end 186.923212 119.802856) (width 0.2) (layer "F.Cu") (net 8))
 (segment (start 184.851786 123.083586) (end 185.475 123.7068) (width 0.2) (layer "F.Cu") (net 49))
 (segment (start 185.475 123.7068) (end 185.475 124.613249) (width 0.2) (layer "F.Cu") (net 49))
 (segment (start 185.475 124.613249) (end 185.75 124.888249) (width 0.2) (layer "F.Cu") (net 49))
 (segment (start 185.257142 119.3975) (end 184.851786 119.802856) (width 0.2) (layer "F.Cu") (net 49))
 (segment (start 184.851786 119.802856) (end 184.851786 123.083586) (width 0.2) (layer "F.Cu") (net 49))
 (segment (start 185.75 124.888249) (end 185.75 126.83825) (width 0.2) (layer "F.Cu") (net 49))
 (segment (start 184.401784 123.269984) (end 185.025 123.8932) (width 0.2) (layer "F.Cu") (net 47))
 (segment (start 183.996428 119.3975) (end 184.401784 119.802856) (width 0.2) (layer "F.Cu") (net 47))
 (segment (start 184.75 124.888249) (end 184.75 126.83825) (width 0.2) (layer "F.Cu") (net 47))
 (segment (start 184.401784 119.802856) (end 184.401784 123.269984) (width 0.2) (layer "F.Cu") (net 47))
 (segment (start 185.025 124.613249) (end 184.75 124.888249) (width 0.2) (layer "F.Cu") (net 47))
 (segment (start 185.025 123.8932) (end 185.025 124.613249) (width 0.2) (layer "F.Cu") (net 47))
 (segment (start 182.330358 122.500409) (end 182.330358 119.802856) (width 0.2) (layer "F.Cu") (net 2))
 (segment (start 184.25 124.888249) (end 183.975 124.613249) (width 0.2) (layer "F.Cu") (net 2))
 (segment (start 183.975 124.613249) (end 183.975 124.145051) (width 0.2) (layer "F.Cu") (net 2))
 (segment (start 184.25 126.83825) (end 184.25 124.888249) (width 0.2) (layer "F.Cu") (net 2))
 (segment (start 182.330358 119.802856) (end 182.735714 119.3975) (width 0.2) (layer "F.Cu") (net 2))
 (segment (start 183.975 124.145051) (end 182.330358 122.500409) (width 0.2) (layer "F.Cu") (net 2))
 (segment (start 181.880356 119.802856) (end 181.475 119.3975) (width 0.2) (layer "F.Cu") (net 10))
 (segment (start 181.880356 122.686807) (end 181.880356 119.802856) (width 0.2) (layer "F.Cu") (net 10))
 (segment (start 183.525 124.331451) (end 181.880356 122.686807) (width 0.2) (layer "F.Cu") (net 10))
 (segment (start 183.25 126.83825) (end 183.25 124.888249) (width 0.2) (layer "F.Cu") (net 10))
 (segment (start 183.525 124.613249) (end 183.525 124.331451) (width 0.2) (layer "F.Cu") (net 10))
 (segment (start 183.25 124.888249) (end 183.525 124.613249) (width 0.2) (layer "F.Cu") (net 10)))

